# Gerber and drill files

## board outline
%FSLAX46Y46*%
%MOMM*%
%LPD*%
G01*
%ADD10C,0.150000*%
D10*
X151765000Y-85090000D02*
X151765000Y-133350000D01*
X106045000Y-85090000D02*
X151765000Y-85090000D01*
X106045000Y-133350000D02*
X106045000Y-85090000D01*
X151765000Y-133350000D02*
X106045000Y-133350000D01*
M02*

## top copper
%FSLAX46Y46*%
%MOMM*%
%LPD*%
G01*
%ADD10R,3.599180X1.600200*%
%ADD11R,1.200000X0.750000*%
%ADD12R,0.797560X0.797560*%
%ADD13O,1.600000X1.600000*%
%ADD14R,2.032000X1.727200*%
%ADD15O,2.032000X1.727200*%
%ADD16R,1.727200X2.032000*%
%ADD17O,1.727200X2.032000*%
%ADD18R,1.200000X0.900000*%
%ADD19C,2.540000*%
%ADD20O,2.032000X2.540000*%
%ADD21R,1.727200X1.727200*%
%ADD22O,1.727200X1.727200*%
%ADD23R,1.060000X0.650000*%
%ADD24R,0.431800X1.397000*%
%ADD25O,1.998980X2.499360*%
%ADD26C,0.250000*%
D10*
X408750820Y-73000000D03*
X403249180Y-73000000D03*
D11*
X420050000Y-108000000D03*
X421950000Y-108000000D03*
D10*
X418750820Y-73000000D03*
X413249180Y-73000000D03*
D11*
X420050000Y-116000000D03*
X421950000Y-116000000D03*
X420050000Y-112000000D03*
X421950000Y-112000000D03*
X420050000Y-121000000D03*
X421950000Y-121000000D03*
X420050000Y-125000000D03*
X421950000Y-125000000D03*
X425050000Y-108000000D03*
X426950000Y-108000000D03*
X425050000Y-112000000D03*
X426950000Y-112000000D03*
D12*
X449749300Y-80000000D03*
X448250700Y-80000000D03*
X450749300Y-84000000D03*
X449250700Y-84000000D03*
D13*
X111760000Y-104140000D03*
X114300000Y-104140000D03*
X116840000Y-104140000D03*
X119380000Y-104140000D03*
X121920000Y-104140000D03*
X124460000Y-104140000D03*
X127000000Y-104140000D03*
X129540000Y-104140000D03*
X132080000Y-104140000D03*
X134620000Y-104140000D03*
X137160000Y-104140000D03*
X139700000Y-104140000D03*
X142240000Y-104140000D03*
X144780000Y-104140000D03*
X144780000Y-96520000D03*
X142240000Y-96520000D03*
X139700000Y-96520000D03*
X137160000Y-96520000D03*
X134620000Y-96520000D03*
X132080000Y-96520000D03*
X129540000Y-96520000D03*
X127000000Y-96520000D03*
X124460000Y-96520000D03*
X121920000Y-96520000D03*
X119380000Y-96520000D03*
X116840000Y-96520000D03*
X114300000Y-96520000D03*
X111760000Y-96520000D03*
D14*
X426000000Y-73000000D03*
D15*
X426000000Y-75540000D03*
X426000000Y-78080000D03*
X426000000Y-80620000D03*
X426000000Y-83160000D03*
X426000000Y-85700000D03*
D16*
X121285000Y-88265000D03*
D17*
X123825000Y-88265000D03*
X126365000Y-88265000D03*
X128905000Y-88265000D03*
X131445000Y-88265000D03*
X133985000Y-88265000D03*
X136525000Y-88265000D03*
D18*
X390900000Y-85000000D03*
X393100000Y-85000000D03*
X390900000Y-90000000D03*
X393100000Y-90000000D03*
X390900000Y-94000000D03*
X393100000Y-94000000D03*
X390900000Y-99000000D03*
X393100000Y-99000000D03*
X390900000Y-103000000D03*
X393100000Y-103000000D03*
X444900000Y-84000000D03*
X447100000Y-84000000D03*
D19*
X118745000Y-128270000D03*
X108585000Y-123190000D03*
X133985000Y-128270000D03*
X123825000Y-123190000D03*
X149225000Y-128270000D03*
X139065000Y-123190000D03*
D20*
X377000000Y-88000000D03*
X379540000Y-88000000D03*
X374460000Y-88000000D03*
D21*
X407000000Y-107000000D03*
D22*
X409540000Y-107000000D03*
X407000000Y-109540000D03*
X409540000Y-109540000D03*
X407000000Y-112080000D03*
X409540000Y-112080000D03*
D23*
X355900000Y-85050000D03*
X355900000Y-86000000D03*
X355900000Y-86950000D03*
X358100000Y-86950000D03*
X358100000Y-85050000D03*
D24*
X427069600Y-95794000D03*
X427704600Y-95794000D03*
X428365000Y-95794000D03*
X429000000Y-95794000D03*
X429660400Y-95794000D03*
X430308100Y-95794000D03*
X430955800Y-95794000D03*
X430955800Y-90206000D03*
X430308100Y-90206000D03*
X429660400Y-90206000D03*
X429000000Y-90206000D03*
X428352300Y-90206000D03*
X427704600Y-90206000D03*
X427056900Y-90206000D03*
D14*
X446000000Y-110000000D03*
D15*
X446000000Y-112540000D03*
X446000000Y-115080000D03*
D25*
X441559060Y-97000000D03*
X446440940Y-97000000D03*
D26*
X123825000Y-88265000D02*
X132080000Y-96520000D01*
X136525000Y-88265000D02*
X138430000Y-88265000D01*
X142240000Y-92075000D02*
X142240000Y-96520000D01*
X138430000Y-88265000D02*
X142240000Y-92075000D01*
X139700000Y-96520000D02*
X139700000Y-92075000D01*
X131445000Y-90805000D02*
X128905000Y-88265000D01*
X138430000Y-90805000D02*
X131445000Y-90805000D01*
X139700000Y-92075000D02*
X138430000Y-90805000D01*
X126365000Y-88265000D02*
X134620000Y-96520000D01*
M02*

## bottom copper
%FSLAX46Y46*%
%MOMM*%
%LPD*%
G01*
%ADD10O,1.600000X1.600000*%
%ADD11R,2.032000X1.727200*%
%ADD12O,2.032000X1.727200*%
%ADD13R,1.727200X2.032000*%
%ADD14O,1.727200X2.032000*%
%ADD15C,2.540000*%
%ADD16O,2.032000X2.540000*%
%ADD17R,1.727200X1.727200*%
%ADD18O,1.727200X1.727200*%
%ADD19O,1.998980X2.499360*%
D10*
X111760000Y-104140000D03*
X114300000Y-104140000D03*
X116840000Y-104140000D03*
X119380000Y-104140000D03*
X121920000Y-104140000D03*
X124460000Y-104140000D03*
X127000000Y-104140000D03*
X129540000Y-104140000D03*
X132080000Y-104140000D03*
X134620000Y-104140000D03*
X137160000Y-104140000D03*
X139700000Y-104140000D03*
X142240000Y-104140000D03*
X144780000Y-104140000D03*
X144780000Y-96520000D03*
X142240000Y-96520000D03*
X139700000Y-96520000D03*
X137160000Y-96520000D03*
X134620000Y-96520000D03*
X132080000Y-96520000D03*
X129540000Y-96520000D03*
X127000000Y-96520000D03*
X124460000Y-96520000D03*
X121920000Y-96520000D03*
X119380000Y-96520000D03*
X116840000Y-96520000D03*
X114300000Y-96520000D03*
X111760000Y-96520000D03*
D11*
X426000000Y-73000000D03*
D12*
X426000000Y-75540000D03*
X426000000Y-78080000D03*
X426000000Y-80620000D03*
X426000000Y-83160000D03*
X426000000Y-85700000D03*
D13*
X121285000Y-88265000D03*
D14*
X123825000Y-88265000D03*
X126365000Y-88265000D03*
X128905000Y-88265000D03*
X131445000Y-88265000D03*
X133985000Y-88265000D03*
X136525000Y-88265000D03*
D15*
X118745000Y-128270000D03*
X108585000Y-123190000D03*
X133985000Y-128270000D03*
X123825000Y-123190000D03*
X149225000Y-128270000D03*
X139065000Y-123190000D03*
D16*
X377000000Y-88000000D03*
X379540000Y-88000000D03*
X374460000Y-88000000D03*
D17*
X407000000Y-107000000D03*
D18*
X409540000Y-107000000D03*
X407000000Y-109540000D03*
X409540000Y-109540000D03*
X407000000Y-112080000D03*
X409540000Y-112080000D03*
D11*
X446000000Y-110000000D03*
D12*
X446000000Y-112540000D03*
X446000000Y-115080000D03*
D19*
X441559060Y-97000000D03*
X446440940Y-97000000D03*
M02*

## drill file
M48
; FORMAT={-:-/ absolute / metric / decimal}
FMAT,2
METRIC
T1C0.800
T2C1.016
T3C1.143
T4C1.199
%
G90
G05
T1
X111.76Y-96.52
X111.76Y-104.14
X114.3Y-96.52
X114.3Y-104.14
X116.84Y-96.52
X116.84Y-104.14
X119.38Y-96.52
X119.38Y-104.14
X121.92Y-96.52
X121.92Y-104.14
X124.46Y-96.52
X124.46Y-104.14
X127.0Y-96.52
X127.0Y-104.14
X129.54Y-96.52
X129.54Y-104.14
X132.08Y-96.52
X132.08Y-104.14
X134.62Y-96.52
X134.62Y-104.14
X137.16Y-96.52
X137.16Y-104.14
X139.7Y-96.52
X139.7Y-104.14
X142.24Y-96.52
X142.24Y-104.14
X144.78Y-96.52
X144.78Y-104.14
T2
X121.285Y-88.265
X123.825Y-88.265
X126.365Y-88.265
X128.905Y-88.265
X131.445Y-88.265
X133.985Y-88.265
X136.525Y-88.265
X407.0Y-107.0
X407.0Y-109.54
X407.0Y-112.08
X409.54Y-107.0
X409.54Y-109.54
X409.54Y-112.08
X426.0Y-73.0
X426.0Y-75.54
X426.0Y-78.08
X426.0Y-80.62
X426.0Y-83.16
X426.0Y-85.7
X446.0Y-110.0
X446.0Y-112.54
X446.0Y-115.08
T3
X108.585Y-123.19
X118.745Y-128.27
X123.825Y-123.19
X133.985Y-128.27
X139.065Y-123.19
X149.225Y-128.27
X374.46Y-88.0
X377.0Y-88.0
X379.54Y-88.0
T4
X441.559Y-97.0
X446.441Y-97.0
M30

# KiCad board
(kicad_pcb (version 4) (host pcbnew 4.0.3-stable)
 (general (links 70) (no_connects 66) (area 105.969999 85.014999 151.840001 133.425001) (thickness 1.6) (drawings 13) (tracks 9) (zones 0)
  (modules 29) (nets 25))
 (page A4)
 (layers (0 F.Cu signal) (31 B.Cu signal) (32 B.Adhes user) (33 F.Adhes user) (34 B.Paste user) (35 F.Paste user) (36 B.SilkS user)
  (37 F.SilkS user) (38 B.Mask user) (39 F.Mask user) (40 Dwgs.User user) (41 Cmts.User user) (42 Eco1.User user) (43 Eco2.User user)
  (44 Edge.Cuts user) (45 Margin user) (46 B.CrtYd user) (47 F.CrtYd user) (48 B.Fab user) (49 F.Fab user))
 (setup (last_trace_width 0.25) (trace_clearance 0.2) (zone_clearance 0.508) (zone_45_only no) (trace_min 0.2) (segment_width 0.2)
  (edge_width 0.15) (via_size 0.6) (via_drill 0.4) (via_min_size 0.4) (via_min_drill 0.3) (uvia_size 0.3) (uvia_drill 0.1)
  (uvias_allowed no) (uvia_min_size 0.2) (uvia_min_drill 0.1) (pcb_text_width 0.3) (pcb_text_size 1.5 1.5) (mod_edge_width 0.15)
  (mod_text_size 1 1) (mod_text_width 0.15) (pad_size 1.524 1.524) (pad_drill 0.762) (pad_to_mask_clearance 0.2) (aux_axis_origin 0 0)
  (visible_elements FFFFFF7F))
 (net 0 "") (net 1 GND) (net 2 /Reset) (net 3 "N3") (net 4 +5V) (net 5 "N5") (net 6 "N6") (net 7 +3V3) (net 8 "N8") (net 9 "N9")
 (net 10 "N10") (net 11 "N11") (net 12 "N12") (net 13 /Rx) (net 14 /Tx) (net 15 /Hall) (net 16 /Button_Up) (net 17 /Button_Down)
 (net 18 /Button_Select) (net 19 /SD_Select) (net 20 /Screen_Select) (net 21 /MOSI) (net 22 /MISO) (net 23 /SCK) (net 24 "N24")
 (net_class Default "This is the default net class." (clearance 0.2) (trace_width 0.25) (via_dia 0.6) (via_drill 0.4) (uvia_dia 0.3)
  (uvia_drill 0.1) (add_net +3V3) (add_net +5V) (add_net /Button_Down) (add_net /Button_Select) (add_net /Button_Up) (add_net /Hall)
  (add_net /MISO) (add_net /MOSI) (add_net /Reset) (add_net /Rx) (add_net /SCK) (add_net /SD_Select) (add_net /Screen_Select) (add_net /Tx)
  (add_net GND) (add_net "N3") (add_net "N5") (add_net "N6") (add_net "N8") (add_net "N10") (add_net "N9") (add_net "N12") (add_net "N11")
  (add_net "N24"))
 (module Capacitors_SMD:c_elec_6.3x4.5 (layer F.Cu) (at 406 73)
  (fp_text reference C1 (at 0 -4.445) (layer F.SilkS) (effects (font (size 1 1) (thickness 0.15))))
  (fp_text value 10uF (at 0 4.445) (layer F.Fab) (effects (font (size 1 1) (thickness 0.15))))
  (pad 1 smd rect (at 2.75082 0) (size 3.59918 1.6002) (layers F.Cu F.Paste F.Mask))
  (pad 2 smd rect (at -2.75082 0) (size 3.59918 1.6002) (layers F.Cu F.Paste F.Mask) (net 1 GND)))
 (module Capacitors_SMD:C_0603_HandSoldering (layer F.Cu) (at 421 108)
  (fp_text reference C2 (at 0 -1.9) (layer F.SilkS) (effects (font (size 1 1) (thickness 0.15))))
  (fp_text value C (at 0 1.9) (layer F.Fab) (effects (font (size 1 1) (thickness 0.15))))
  (pad 1 smd rect (at -0.95 0) (size 1.2 0.75) (layers F.Cu F.Paste F.Mask) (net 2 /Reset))
  (pad 2 smd rect (at 0.95 0) (size 1.2 0.75) (layers F.Cu F.Paste F.Mask) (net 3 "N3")))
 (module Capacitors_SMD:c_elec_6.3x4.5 (layer F.Cu) (at 416 73)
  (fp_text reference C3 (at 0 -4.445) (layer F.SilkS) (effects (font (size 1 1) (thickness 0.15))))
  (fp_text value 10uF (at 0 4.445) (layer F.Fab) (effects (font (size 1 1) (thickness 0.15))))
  (pad 1 smd rect (at 2.75082 0) (size 3.59918 1.6002) (layers F.Cu F.Paste F.Mask) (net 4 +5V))
  (pad 2 smd rect (at -2.75082 0) (size 3.59918 1.6002) (layers F.Cu F.Paste F.Mask) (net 1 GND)))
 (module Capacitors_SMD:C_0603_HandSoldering (layer F.Cu) (at 421 116)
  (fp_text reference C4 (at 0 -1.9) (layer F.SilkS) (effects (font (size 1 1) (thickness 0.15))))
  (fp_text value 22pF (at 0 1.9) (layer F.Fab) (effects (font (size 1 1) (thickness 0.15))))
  (pad 1 smd rect (at -0.95 0) (size 1.2 0.75) (layers F.Cu F.Paste F.Mask) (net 1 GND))
  (pad 2 smd rect (at 0.95 0) (size 1.2 0.75) (layers F.Cu F.Paste F.Mask) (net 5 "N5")))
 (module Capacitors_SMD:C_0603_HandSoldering (layer F.Cu) (at 421 112)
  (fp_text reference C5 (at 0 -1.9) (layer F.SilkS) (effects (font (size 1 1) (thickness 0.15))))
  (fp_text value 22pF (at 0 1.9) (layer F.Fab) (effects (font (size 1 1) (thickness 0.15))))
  (pad 1 smd rect (at -0.95 0) (size 1.2 0.75) (layers F.Cu F.Paste F.Mask) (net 1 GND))
  (pad 2 smd rect (at 0.95 0) (size 1.2 0.75) (layers F.Cu F.Paste F.Mask) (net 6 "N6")))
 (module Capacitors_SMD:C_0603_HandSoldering (layer F.Cu) (at 421 121)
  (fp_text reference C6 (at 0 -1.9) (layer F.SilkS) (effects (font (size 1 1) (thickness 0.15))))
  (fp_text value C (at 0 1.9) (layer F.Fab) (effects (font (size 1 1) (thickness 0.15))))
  (pad 1 smd rect (at -0.95 0) (size 1.2 0.75) (layers F.Cu F.Paste F.Mask) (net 4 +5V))
  (pad 2 smd rect (at 0.95 0) (size 1.2 0.75) (layers F.Cu F.Paste F.Mask) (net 1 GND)))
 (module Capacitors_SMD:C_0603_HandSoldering (layer F.Cu) (at 421 125)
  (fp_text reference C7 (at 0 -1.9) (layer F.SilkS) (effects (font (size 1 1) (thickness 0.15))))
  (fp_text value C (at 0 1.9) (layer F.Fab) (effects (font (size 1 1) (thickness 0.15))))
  (pad 1 smd rect (at -0.95 0) (size 1.2 0.75) (layers F.Cu F.Paste F.Mask) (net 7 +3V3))
  (pad 2 smd rect (at 0.95 0) (size 1.2 0.75) (layers F.Cu F.Paste F.Mask) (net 1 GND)))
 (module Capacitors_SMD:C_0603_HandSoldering (layer F.Cu) (at 426 108)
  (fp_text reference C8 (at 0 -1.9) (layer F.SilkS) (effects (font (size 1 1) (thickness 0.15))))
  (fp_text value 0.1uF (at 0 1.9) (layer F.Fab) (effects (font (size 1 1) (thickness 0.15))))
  (pad 1 smd rect (at -0.95 0) (size 1.2 0.75) (layers F.Cu F.Paste F.Mask) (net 4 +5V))
  (pad 2 smd rect (at 0.95 0) (size 1.2 0.75) (layers F.Cu F.Paste F.Mask) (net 1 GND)))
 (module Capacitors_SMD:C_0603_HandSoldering (layer F.Cu) (at 426 112)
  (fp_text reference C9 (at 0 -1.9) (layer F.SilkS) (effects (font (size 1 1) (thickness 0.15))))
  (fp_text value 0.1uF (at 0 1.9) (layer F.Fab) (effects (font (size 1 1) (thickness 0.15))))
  (pad 1 smd rect (at -0.95 0) (size 1.2 0.75) (layers F.Cu F.Paste F.Mask) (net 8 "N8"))
  (pad 2 smd rect (at 0.95 0) (size 1.2 0.75) (layers F.Cu F.Paste F.Mask) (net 1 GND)))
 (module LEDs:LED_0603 (layer F.Cu) (at 449 80)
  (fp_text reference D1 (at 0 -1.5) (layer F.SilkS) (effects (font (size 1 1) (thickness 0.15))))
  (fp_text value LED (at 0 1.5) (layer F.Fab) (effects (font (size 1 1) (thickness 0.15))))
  (pad 2 smd rect (at 0.7493 0 180) (size 0.79756 0.79756) (layers F.Cu F.Paste F.Mask) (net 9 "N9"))
  (pad 1 smd rect (at -0.7493 0 180) (size 0.79756 0.79756) (layers F.Cu F.Paste F.Mask) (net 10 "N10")))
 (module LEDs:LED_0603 (layer F.Cu) (at 450 84)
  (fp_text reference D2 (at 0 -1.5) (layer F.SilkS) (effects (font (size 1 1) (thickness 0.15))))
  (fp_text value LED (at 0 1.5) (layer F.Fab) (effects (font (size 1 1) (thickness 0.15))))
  (pad 2 smd rect (at 0.7493 0 180) (size 0.79756 0.79756) (layers F.Cu F.Paste F.Mask) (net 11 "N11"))
  (pad 1 smd rect (at -0.7493 0 180) (size 0.79756 0.79756) (layers F.Cu F.Paste F.Mask) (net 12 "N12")))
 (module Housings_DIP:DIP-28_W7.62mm (layer F.Cu) (at 111.76 104.14 90)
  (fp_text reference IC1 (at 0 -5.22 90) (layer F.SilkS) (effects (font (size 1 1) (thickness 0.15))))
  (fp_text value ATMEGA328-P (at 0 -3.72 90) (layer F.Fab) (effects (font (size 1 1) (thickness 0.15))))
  (pad 1 thru_hole oval (at 0 0 90) (size 1.6 1.6) (drill 0.8) (layers *.Cu *.Mask F.SilkS) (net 2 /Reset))
  (pad 2 thru_hole oval (at 0 2.54 90) (size 1.6 1.6) (drill 0.8) (layers *.Cu *.Mask F.SilkS) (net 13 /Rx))
  (pad 3 thru_hole oval (at 0 5.08 90) (size 1.6 1.6) (drill 0.8) (layers *.Cu *.Mask F.SilkS) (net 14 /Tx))
  (pad 4 thru_hole oval (at 0 7.62 90) (size 1.6 1.6) (drill 0.8) (layers *.Cu *.Mask F.SilkS) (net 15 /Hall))
  (pad 5 thru_hole oval (at 0 10.16 90) (size 1.6 1.6) (drill 0.8) (layers *.Cu *.Mask F.SilkS))
  (pad 6 thru_hole oval (at 0 12.7 90) (size 1.6 1.6) (drill 0.8) (layers *.Cu *.Mask F.SilkS) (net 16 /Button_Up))
  (pad 7 thru_hole oval (at 0 15.24 90) (size 1.6 1.6) (drill 0.8) (layers *.Cu *.Mask F.SilkS) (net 4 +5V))
  (pad 8 thru_hole oval (at 0 17.78 90) (size 1.6 1.6) (drill 0.8) (layers *.Cu *.Mask F.SilkS) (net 1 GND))
  (pad 9 thru_hole oval (at 0 20.32 90) (size 1.6 1.6) (drill 0.8) (layers *.Cu *.Mask F.SilkS) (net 5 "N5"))
  (pad 10 thru_hole oval (at 0 22.86 90) (size 1.6 1.6) (drill 0.8) (layers *.Cu *.Mask F.SilkS) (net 6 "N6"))
  (pad 11 thru_hole oval (at 0 25.4 90) (size 1.6 1.6) (drill 0.8) (layers *.Cu *.Mask F.SilkS) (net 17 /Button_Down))
  (pad 12 thru_hole oval (at 0 27.94 90) (size 1.6 1.6) (drill 0.8) (layers *.Cu *.Mask F.SilkS) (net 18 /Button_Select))
  (pad 13 thru_hole oval (at 0 30.48 90) (size 1.6 1.6) (drill 0.8) (layers *.Cu *.Mask F.SilkS) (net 9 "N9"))
  (pad 14 thru_hole oval (at 0 33.02 90) (size 1.6 1.6) (drill 0.8) (layers *.Cu *.Mask F.SilkS))
  (pad 15 thru_hole oval (at 7.62 33.02 90) (size 1.6 1.6) (drill 0.8) (layers *.Cu *.Mask F.SilkS) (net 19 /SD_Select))
  (pad 16 thru_hole oval (at 7.62 30.48 90) (size 1.6 1.6) (drill 0.8) (layers *.Cu *.Mask F.SilkS) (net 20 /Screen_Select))
  (pad 17 thru_hole oval (at 7.62 27.94 90) (size 1.6 1.6) (drill 0.8) (layers *.Cu *.Mask F.SilkS) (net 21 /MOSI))
  (pad 18 thru_hole oval (at 7.62 25.4 90) (size 1.6 1.6) (drill 0.8) (layers *.Cu *.Mask F.SilkS) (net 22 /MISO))
  (pad 19 thru_hole oval (at 7.62 22.86 90) (size 1.6 1.6) (drill 0.8) (layers *.Cu *.Mask F.SilkS) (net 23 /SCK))
  (pad 20 thru_hole oval (at 7.62 20.32 90) (size 1.6 1.6) (drill 0.8) (layers *.Cu *.Mask F.SilkS) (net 4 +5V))
  (pad 21 thru_hole oval (at 7.62 17.78 90) (size 1.6 1.6) (drill 0.8) (layers *.Cu *.Mask F.SilkS) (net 8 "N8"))
  (pad 22 thru_hole oval (at 7.62 15.24 90) (size 1.6 1.6) (drill 0.8) (layers *.Cu *.Mask F.SilkS) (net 1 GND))
  (pad 23 thru_hole oval (at 7.62 12.7 90) (size 1.6 1.6) (drill 0.8) (layers *.Cu *.Mask F.SilkS))
  (pad 24 thru_hole oval (at 7.62 10.16 90) (size 1.6 1.6) (drill 0.8) (layers *.Cu *.Mask F.SilkS))
  (pad 25 thru_hole oval (at 7.62 7.62 90) (size 1.6 1.6) (drill 0.8) (layers *.Cu *.Mask F.SilkS))
  (pad 26 thru_hole oval (at 7.62 5.08 90) (size 1.6 1.6) (drill 0.8) (layers *.Cu *.Mask F.SilkS))
  (pad 27 thru_hole oval (at 7.62 2.54 90) (size 1.6 1.6) (drill 0.8) (layers *.Cu *.Mask F.SilkS))
  (pad 28 thru_hole oval (at 7.62 0 90) (size 1.6 1.6) (drill 0.8) (layers *.Cu *.Mask F.SilkS)))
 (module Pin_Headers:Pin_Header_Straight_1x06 (layer F.Cu) (at 426 73)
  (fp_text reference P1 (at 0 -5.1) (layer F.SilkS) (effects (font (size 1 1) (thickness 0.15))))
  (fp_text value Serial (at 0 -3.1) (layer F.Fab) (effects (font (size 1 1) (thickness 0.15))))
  (pad 1 thru_hole rect (at 0 0) (size 2.032 1.7272) (drill 1.016) (layers *.Cu *.Mask F.SilkS) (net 1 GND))
  (pad 2 thru_hole oval (at 0 2.54) (size 2.032 1.7272) (drill 1.016) (layers *.Cu *.Mask F.SilkS))
  (pad 3 thru_hole oval (at 0 5.08) (size 2.032 1.7272) (drill 1.016) (layers *.Cu *.Mask F.SilkS) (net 4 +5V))
  (pad 4 thru_hole oval (at 0 7.62) (size 2.032 1.7272) (drill 1.016) (layers *.Cu *.Mask F.SilkS) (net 13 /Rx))
  (pad 5 thru_hole oval (at 0 10.16) (size 2.032 1.7272) (drill 1.016) (layers *.Cu *.Mask F.SilkS) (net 14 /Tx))
  (pad 6 thru_hole oval (at 0 12.7) (size 2.032 1.7272) (drill 1.016) (layers *.Cu *.Mask F.SilkS) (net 3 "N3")))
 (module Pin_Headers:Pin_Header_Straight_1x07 (layer F.Cu) (at 121.285 88.265 90)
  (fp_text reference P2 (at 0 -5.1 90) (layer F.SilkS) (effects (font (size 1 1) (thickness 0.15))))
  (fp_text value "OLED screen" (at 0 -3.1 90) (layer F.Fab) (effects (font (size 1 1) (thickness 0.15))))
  (pad 1 thru_hole rect (at 0 0 90) (size 2.032 1.7272) (drill 1.016) (layers *.Cu *.Mask F.SilkS) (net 1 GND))
  (pad 2 thru_hole oval (at 0 2.54 90) (size 2.032 1.7272) (drill 1.016) (layers *.Cu *.Mask F.SilkS) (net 4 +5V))
  (pad 3 thru_hole oval (at 0 5.08 90) (size 2.032 1.7272) (drill 1.016) (layers *.Cu *.Mask F.SilkS) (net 23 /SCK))
  (pad 4 thru_hole oval (at 0 7.62 90) (size 2.032 1.7272) (drill 1.016) (layers *.Cu *.Mask F.SilkS) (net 21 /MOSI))
  (pad 5 thru_hole oval (at 0 10.16 90) (size 2.032 1.7272) (drill 1.016) (layers *.Cu *.Mask F.SilkS))
  (pad 6 thru_hole oval (at 0 12.7 90) (size 2.032 1.7272) (drill 1.016) (layers *.Cu *.Mask F.SilkS))
  (pad 7 thru_hole oval (at 0 15.24 90) (size 2.032 1.7272) (drill 1.016) (layers *.Cu *.Mask F.SilkS) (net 20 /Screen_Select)))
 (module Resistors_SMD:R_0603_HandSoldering (layer F.Cu) (at 392 85)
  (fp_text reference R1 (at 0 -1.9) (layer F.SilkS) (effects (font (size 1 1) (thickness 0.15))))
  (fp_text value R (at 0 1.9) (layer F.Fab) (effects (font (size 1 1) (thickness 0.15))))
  (pad 1 smd rect (at -1.1 0) (size 1.2 0.9) (layers F.Cu F.Paste F.Mask) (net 4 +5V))
  (pad 2 smd rect (at 1.1 0) (size 1.2 0.9) (layers F.Cu F.Paste F.Mask) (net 16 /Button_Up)))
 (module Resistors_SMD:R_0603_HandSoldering (layer F.Cu) (at 392 90)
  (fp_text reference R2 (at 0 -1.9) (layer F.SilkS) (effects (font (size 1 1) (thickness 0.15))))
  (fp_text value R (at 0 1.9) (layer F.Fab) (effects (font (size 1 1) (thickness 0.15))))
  (pad 1 smd rect (at -1.1 0) (size 1.2 0.9) (layers F.Cu F.Paste F.Mask) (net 4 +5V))
  (pad 2 smd rect (at 1.1 0) (size 1.2 0.9) (layers F.Cu F.Paste F.Mask) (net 18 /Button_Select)))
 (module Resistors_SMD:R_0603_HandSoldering (layer F.Cu) (at 392 94)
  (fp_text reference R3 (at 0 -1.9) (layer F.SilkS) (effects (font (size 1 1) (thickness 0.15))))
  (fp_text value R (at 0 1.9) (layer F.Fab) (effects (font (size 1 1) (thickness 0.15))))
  (pad 1 smd rect (at -1.1 0) (size 1.2 0.9) (layers F.Cu F.Paste F.Mask) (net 4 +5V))
  (pad 2 smd rect (at 1.1 0) (size 1.2 0.9) (layers F.Cu F.Paste F.Mask) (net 17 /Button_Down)))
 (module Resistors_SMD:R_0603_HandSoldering (layer F.Cu) (at 392 99)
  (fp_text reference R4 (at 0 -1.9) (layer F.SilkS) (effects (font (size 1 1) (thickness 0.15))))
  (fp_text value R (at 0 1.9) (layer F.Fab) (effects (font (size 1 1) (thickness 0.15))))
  (pad 1 smd rect (at -1.1 0) (size 1.2 0.9) (layers F.Cu F.Paste F.Mask) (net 10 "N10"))
  (pad 2 smd rect (at 1.1 0) (size 1.2 0.9) (layers F.Cu F.Paste F.Mask) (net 1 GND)))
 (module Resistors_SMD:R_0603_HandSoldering (layer F.Cu) (at 392 103)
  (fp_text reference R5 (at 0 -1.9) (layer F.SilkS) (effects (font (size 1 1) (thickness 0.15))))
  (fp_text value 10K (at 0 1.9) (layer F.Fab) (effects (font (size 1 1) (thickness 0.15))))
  (pad 1 smd rect (at -1.1 0) (size 1.2 0.9) (layers F.Cu F.Paste F.Mask) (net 4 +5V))
  (pad 2 smd rect (at 1.1 0) (size 1.2 0.9) (layers F.Cu F.Paste F.Mask) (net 15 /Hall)))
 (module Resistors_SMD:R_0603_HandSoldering (layer F.Cu) (at 446 84)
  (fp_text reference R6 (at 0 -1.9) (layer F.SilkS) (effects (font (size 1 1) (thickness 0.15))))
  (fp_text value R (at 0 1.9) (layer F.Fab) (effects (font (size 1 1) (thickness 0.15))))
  (pad 1 smd rect (at -1.1 0) (size 1.2 0.9) (layers F.Cu F.Paste F.Mask) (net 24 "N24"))
  (pad 2 smd rect (at 1.1 0) (size 1.2 0.9) (layers F.Cu F.Paste F.Mask) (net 12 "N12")))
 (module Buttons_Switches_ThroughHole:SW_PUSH (layer F.Cu) (at 113.665 125.73 180)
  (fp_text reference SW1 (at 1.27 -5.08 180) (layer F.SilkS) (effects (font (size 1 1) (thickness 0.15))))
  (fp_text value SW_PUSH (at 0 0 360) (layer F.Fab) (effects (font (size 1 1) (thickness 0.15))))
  (pad 1 thru_hole circle (at -5.08 -2.54 180) (size 2.54 2.54) (drill 1.143) (layers *.Cu *.Mask F.SilkS) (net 1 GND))
  (pad 2 thru_hole circle (at 5.08 2.54 180) (size 2.54 2.54) (drill 1.143) (layers *.Cu *.Mask F.SilkS) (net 16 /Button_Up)))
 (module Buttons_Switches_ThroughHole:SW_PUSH (layer F.Cu) (at 128.905 125.73 180)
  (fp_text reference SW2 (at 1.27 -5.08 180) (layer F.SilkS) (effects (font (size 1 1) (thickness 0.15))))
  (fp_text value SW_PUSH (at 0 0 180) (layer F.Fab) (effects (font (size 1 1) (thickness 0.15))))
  (pad 1 thru_hole circle (at -5.08 -2.54 180) (size 2.54 2.54) (drill 1.143) (layers *.Cu *.Mask F.SilkS) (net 1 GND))
  (pad 2 thru_hole circle (at 5.08 2.54 180) (size 2.54 2.54) (drill 1.143) (layers *.Cu *.Mask F.SilkS) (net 18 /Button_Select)))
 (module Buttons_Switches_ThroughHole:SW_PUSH (layer F.Cu) (at 144.145 125.73 180)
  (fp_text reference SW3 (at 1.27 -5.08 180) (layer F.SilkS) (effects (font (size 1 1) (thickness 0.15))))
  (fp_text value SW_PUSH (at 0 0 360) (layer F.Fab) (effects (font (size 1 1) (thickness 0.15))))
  (pad 1 thru_hole circle (at -5.08 -2.54 180) (size 2.54 2.54) (drill 1.143) (layers *.Cu *.Mask F.SilkS) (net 1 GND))
  (pad 2 thru_hole circle (at 5.08 2.54 180) (size 2.54 2.54) (drill 1.143) (layers *.Cu *.Mask F.SilkS) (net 17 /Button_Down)))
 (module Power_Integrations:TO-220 (layer F.Cu) (at 377 88)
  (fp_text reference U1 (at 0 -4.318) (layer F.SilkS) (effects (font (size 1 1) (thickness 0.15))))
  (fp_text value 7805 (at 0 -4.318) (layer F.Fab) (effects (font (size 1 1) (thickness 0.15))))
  (pad 2 thru_hole oval (at 0 0) (size 2.032 2.54) (drill 1.143) (layers *.Cu *.Mask F.SilkS))
  (pad 3 thru_hole oval (at 2.54 0) (size 2.032 2.54) (drill 1.143) (layers *.Cu *.Mask F.SilkS))
  (pad 1 thru_hole oval (at -2.54 0) (size 2.032 2.54) (drill 1.143) (layers *.Cu *.Mask F.SilkS)))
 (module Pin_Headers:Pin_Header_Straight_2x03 (layer F.Cu) (at 407 107)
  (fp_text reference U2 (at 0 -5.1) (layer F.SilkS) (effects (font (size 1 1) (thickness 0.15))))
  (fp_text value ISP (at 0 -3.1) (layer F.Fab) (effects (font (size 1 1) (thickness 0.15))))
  (pad 1 thru_hole rect (at 0 0) (size 1.7272 1.7272) (drill 1.016) (layers *.Cu *.Mask F.SilkS) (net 22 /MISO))
  (pad 2 thru_hole oval (at 2.54 0) (size 1.7272 1.7272) (drill 1.016) (layers *.Cu *.Mask F.SilkS) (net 4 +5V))
  (pad 3 thru_hole oval (at 0 2.54) (size 1.7272 1.7272) (drill 1.016) (layers *.Cu *.Mask F.SilkS) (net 23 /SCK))
  (pad 4 thru_hole oval (at 2.54 2.54) (size 1.7272 1.7272) (drill 1.016) (layers *.Cu *.Mask F.SilkS) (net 21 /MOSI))
  (pad 5 thru_hole oval (at 0 5.08) (size 1.7272 1.7272) (drill 1.016) (layers *.Cu *.Mask F.SilkS) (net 2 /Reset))
  (pad 6 thru_hole oval (at 2.54 5.08) (size 1.7272 1.7272) (drill 1.016) (layers *.Cu *.Mask F.SilkS) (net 1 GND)))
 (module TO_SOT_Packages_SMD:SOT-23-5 (layer F.Cu) (at 357 86)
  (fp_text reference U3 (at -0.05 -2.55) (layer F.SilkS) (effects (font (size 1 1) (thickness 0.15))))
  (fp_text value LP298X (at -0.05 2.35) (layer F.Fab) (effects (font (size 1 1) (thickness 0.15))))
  (pad 1 smd rect (at -1.1 -0.95) (size 1.06 0.65) (layers F.Cu F.Paste F.Mask) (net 4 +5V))
  (pad 2 smd rect (at -1.1 0) (size 1.06 0.65) (layers F.Cu F.Paste F.Mask) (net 1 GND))
  (pad 3 smd rect (at -1.1 0.95) (size 1.06 0.65) (layers F.Cu F.Paste F.Mask) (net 4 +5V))
  (pad 4 smd rect (at 1.1 0.95) (size 1.06 0.65) (layers F.Cu F.Paste F.Mask))
  (pad 5 smd rect (at 1.1 -0.95) (size 1.06 0.65) (layers F.Cu F.Paste F.Mask) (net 7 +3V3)))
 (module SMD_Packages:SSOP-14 (layer F.Cu) (at 429 93)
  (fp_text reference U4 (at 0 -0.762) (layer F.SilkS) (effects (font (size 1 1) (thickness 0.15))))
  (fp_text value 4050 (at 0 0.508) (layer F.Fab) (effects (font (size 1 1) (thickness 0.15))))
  (pad 1 smd rect (at -1.9304 2.794) (size 0.4318 1.397) (layers F.Cu F.Paste F.Mask) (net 7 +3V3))
  (pad 2 smd rect (at -1.2954 2.794) (size 0.4318 1.397) (layers F.Cu F.Paste F.Mask) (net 24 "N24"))
  (pad 3 smd rect (at -0.635 2.794) (size 0.4318 1.397) (layers F.Cu F.Paste F.Mask) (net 19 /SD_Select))
  (pad 4 smd rect (at 0 2.794) (size 0.4318 1.397) (layers F.Cu F.Paste F.Mask))
  (pad 5 smd rect (at 0.6604 2.794) (size 0.4318 1.397) (layers F.Cu F.Paste F.Mask) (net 21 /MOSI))
  (pad 6 smd rect (at 1.3081 2.794) (size 0.4318 1.397) (layers F.Cu F.Paste F.Mask))
  (pad 7 smd rect (at 1.9558 2.794) (size 0.4318 1.397) (layers F.Cu F.Paste F.Mask) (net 23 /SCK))
  (pad 8 smd rect (at 1.9558 -2.794) (size 0.4318 1.397) (layers F.Cu F.Paste F.Mask) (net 1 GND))
  (pad 9 smd rect (at 1.3081 -2.794) (size 0.4318 1.397) (layers F.Cu F.Paste F.Mask) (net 23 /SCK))
  (pad 10 smd rect (at 0.6604 -2.794) (size 0.4318 1.397) (layers F.Cu F.Paste F.Mask) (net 11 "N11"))
  (pad 11 smd rect (at 0 -2.794) (size 0.4318 1.397) (layers F.Cu F.Paste F.Mask) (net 1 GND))
  (pad 12 smd rect (at -0.6477 -2.794) (size 0.4318 1.397) (layers F.Cu F.Paste F.Mask))
  (pad 13 smd rect (at -1.2954 -2.794) (size 0.4318 1.397) (layers F.Cu F.Paste F.Mask))
  (pad 14 smd rect (at -1.9431 -2.794) (size 0.4318 1.397) (layers F.Cu F.Paste F.Mask) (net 1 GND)))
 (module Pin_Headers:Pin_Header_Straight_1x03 (layer F.Cu) (at 446 110)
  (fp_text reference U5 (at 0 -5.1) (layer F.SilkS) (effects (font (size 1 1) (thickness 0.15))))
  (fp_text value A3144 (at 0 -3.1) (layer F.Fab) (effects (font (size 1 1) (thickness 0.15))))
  (pad 1 thru_hole rect (at 0 0) (size 2.032 1.7272) (drill 1.016) (layers *.Cu *.Mask F.SilkS) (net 4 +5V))
  (pad 2 thru_hole oval (at 0 2.54) (size 2.032 1.7272) (drill 1.016) (layers *.Cu *.Mask F.SilkS) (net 1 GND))
  (pad 3 thru_hole oval (at 0 5.08) (size 2.032 1.7272) (drill 1.016) (layers *.Cu *.Mask F.SilkS) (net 15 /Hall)))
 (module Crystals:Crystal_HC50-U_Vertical (layer F.Cu) (at 444 97)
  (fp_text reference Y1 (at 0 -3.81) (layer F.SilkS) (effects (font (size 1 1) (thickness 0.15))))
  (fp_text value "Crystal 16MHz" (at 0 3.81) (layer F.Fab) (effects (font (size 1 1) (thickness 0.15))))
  (pad 1 thru_hole oval (at -2.44094 0) (size 1.99898 2.49936) (drill 1.19888) (layers *.Cu *.Mask F.SilkS) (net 6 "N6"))
  (pad 2 thru_hole oval (at 2.44094 0) (size 1.99898 2.49936) (drill 1.19888) (layers *.Cu *.Mask F.SilkS) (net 5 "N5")))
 (gr_line (start 151.765 85.09) (end 151.765 133.35) (layer Edge.Cuts) (width 0.15))
 (gr_line (start 106.045 85.09) (end 151.765 85.09) (layer Edge.Cuts) (width 0.15))
 (gr_line (start 106.045 133.35) (end 106.045 85.09) (layer Edge.Cuts) (width 0.15))
 (gr_line (start 151.765 133.35) (end 106.045 133.35) (layer Edge.Cuts) (width 0.15))
 (segment (start 123.825 88.265) (end 132.08 96.52) (width 0.25) (layer F.Cu) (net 4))
 (segment (start 136.525 88.265) (end 138.43 88.265) (width 0.25) (layer F.Cu) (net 20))
 (segment (start 142.24 92.075) (end 142.24 96.52) (width 0.25) (layer F.Cu) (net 20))
 (segment (start 138.43 88.265) (end 142.24 92.075) (width 0.25) (layer F.Cu) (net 20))
 (segment (start 139.7 96.52) (end 139.7 92.075) (width 0.25) (layer F.Cu) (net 21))
 (segment (start 131.445 90.805) (end 128.905 88.265) (width 0.25) (layer F.Cu) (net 21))
 (segment (start 138.43 90.805) (end 131.445 90.805) (width 0.25) (layer F.Cu) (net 21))
 (segment (start 139.7 92.075) (end 138.43 90.805) (width 0.25) (layer F.Cu) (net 21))
 (segment (start 126.365 88.265) (end 134.62 96.52) (width 0.25) (layer F.Cu) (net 23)))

